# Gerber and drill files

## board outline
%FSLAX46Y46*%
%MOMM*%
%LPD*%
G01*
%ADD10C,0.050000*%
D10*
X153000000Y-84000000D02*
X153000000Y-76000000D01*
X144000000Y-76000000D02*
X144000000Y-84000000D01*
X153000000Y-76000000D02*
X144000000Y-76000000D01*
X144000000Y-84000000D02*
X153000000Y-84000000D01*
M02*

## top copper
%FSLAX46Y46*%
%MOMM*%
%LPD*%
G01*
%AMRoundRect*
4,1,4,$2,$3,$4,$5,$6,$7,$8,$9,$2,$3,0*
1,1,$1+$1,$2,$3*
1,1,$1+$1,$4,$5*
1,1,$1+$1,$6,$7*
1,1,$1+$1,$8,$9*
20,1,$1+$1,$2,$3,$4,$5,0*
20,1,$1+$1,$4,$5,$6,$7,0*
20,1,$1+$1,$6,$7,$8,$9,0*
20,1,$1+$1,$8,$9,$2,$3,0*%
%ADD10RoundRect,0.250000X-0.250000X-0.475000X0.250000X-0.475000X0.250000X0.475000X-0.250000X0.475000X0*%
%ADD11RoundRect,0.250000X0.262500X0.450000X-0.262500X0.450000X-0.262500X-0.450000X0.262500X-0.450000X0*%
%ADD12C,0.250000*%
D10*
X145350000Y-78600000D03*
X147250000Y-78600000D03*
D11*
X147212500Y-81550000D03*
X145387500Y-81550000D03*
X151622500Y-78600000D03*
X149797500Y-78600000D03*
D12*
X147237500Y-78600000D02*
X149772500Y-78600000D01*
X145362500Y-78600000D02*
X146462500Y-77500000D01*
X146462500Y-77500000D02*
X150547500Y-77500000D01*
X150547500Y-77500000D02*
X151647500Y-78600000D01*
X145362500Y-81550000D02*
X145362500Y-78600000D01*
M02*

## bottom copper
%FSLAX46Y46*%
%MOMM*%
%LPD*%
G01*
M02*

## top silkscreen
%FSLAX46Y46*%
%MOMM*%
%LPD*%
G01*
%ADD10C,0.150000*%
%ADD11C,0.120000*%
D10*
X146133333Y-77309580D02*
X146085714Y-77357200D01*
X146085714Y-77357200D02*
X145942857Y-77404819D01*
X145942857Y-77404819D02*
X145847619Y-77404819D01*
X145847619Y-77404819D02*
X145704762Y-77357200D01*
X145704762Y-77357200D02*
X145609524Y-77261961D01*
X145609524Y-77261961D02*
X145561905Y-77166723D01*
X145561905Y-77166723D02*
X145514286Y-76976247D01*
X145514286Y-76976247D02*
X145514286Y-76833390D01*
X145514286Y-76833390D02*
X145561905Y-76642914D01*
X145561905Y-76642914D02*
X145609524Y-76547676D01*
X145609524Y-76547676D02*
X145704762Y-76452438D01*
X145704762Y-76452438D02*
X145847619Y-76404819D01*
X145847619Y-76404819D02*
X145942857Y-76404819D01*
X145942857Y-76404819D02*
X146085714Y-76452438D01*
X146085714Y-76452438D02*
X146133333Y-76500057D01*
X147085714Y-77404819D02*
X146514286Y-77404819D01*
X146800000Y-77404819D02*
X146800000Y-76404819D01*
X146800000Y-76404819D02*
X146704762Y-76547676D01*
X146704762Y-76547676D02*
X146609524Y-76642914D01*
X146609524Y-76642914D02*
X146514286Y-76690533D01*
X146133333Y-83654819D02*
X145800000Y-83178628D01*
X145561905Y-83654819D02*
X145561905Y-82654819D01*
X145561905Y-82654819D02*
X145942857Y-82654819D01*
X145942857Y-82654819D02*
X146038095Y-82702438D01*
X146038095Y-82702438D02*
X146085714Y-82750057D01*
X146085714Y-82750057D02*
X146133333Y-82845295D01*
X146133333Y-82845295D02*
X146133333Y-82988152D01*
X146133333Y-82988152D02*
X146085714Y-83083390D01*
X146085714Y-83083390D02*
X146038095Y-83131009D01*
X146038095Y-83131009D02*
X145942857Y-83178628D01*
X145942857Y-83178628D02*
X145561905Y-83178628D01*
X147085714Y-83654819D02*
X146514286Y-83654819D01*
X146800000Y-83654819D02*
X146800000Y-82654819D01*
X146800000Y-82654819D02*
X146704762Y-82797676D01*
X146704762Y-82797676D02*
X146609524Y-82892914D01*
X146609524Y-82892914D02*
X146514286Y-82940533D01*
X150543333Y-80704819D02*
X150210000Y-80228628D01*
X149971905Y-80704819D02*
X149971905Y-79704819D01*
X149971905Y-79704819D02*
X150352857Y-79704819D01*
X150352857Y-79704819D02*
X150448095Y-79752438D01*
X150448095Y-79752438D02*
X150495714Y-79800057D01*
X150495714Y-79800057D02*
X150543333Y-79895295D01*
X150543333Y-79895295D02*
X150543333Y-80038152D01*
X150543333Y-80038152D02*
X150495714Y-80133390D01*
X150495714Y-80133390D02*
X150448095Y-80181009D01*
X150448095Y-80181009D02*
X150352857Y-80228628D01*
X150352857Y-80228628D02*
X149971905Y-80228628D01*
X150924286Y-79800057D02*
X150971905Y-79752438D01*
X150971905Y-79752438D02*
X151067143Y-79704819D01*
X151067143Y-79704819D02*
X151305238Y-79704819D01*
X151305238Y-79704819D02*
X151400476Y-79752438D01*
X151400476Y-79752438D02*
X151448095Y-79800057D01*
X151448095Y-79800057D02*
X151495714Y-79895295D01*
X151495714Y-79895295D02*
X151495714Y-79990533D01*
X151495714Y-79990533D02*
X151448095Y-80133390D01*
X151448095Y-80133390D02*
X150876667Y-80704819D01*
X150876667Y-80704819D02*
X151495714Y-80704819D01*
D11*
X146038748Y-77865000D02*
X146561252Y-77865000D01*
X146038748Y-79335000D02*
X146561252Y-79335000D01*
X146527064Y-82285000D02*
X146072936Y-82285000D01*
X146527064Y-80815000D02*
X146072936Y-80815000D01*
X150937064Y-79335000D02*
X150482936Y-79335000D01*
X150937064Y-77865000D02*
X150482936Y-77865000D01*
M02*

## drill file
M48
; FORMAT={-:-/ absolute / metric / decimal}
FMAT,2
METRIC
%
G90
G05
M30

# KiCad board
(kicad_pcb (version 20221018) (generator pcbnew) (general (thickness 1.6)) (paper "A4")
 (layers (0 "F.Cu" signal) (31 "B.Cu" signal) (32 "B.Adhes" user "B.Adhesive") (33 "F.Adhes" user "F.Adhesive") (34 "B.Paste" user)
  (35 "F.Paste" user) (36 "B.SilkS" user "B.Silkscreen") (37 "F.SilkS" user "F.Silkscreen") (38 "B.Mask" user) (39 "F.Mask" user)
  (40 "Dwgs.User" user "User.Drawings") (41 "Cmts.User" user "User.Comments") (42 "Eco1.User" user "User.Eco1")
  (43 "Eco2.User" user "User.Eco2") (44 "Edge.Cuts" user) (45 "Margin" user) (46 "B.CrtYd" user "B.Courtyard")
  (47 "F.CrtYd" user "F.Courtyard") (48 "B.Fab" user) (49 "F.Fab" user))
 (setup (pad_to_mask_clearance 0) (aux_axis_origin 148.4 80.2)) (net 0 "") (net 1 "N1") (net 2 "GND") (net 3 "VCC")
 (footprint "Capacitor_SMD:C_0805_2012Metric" (layer "F.Cu") (at 146.3 78.6)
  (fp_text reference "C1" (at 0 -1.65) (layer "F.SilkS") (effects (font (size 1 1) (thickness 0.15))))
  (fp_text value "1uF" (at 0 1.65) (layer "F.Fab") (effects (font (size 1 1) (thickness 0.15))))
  (fp_line (start -0.261252 -0.735) (end 0.261252 -0.735) (stroke (width 0.12) (type solid)) (layer "F.SilkS"))
  (fp_line (start -0.261252 0.735) (end 0.261252 0.735) (stroke (width 0.12) (type solid)) (layer "F.SilkS"))
  (pad "1" smd roundrect (at -0.95 0) (size 1 1.45) (layers "F.Cu" "F.Paste" "F.Mask") (roundrect_rratio 0.25) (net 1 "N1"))
  (pad "2" smd roundrect (at 0.95 0) (size 1 1.45) (layers "F.Cu" "F.Paste" "F.Mask") (roundrect_rratio 0.25) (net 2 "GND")))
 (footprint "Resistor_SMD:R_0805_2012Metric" (layer "F.Cu") (at 146.3 81.55 180)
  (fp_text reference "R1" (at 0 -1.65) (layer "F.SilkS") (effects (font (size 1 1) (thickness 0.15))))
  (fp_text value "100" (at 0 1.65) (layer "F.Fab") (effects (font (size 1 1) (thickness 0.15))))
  (fp_line (start -0.227064 -0.735) (end 0.227064 -0.735) (stroke (width 0.12) (type solid)) (layer "F.SilkS"))
  (fp_line (start -0.227064 0.735) (end 0.227064 0.735) (stroke (width 0.12) (type solid)) (layer "F.SilkS"))
  (pad "1" smd roundrect (at -0.9125 0 180) (size 1.025 1.4) (layers "F.Cu" "F.Paste" "F.Mask") (roundrect_rratio 0.243902) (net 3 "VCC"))
  (pad "2" smd roundrect (at 0.9125 0 180) (size 1.025 1.4) (layers "F.Cu" "F.Paste" "F.Mask") (roundrect_rratio 0.243902) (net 1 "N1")))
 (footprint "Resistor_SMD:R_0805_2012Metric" (layer "F.Cu") (at 150.71 78.6 180)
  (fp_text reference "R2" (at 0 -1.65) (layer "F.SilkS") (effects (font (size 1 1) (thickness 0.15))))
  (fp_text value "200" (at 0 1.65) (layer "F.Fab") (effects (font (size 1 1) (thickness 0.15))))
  (fp_line (start -0.227064 -0.735) (end 0.227064 -0.735) (stroke (width 0.12) (type solid)) (layer "F.SilkS"))
  (fp_line (start -0.227064 0.735) (end 0.227064 0.735) (stroke (width 0.12) (type solid)) (layer "F.SilkS"))
  (pad "1" smd roundrect (at -0.9125 0 180) (size 1.025 1.4) (layers "F.Cu" "F.Paste" "F.Mask") (roundrect_rratio 0.243902) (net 1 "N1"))
  (pad "2" smd roundrect (at 0.9125 0 180) (size 1.025 1.4) (layers "F.Cu" "F.Paste" "F.Mask") (roundrect_rratio 0.243902) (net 2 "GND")))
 (gr_line (start 153 84) (end 153 76) (stroke (width 0.05) (type solid)) (layer "Edge.Cuts"))
 (gr_line (start 144 76) (end 144 84) (stroke (width 0.05) (type solid)) (layer "Edge.Cuts"))
 (gr_line (start 153 76) (end 144 76) (stroke (width 0.05) (type solid)) (layer "Edge.Cuts"))
 (gr_line (start 144 84) (end 153 84) (stroke (width 0.05) (type solid)) (layer "Edge.Cuts"))
 (segment (start 147.2375 78.6) (end 149.7725 78.6) (width 0.25) (layer "F.Cu") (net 2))
 (segment (start 145.3625 78.6) (end 146.4625 77.5) (width 0.25) (layer "F.Cu") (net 1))
 (segment (start 146.4625 77.5) (end 150.5475 77.5) (width 0.25) (layer "F.Cu") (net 1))
 (segment (start 150.5475 77.5) (end 151.6475 78.6) (width 0.25) (layer "F.Cu") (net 1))
 (segment (start 145.3625 81.55) (end 145.3625 78.6) (width 0.25) (layer "F.Cu") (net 1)))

